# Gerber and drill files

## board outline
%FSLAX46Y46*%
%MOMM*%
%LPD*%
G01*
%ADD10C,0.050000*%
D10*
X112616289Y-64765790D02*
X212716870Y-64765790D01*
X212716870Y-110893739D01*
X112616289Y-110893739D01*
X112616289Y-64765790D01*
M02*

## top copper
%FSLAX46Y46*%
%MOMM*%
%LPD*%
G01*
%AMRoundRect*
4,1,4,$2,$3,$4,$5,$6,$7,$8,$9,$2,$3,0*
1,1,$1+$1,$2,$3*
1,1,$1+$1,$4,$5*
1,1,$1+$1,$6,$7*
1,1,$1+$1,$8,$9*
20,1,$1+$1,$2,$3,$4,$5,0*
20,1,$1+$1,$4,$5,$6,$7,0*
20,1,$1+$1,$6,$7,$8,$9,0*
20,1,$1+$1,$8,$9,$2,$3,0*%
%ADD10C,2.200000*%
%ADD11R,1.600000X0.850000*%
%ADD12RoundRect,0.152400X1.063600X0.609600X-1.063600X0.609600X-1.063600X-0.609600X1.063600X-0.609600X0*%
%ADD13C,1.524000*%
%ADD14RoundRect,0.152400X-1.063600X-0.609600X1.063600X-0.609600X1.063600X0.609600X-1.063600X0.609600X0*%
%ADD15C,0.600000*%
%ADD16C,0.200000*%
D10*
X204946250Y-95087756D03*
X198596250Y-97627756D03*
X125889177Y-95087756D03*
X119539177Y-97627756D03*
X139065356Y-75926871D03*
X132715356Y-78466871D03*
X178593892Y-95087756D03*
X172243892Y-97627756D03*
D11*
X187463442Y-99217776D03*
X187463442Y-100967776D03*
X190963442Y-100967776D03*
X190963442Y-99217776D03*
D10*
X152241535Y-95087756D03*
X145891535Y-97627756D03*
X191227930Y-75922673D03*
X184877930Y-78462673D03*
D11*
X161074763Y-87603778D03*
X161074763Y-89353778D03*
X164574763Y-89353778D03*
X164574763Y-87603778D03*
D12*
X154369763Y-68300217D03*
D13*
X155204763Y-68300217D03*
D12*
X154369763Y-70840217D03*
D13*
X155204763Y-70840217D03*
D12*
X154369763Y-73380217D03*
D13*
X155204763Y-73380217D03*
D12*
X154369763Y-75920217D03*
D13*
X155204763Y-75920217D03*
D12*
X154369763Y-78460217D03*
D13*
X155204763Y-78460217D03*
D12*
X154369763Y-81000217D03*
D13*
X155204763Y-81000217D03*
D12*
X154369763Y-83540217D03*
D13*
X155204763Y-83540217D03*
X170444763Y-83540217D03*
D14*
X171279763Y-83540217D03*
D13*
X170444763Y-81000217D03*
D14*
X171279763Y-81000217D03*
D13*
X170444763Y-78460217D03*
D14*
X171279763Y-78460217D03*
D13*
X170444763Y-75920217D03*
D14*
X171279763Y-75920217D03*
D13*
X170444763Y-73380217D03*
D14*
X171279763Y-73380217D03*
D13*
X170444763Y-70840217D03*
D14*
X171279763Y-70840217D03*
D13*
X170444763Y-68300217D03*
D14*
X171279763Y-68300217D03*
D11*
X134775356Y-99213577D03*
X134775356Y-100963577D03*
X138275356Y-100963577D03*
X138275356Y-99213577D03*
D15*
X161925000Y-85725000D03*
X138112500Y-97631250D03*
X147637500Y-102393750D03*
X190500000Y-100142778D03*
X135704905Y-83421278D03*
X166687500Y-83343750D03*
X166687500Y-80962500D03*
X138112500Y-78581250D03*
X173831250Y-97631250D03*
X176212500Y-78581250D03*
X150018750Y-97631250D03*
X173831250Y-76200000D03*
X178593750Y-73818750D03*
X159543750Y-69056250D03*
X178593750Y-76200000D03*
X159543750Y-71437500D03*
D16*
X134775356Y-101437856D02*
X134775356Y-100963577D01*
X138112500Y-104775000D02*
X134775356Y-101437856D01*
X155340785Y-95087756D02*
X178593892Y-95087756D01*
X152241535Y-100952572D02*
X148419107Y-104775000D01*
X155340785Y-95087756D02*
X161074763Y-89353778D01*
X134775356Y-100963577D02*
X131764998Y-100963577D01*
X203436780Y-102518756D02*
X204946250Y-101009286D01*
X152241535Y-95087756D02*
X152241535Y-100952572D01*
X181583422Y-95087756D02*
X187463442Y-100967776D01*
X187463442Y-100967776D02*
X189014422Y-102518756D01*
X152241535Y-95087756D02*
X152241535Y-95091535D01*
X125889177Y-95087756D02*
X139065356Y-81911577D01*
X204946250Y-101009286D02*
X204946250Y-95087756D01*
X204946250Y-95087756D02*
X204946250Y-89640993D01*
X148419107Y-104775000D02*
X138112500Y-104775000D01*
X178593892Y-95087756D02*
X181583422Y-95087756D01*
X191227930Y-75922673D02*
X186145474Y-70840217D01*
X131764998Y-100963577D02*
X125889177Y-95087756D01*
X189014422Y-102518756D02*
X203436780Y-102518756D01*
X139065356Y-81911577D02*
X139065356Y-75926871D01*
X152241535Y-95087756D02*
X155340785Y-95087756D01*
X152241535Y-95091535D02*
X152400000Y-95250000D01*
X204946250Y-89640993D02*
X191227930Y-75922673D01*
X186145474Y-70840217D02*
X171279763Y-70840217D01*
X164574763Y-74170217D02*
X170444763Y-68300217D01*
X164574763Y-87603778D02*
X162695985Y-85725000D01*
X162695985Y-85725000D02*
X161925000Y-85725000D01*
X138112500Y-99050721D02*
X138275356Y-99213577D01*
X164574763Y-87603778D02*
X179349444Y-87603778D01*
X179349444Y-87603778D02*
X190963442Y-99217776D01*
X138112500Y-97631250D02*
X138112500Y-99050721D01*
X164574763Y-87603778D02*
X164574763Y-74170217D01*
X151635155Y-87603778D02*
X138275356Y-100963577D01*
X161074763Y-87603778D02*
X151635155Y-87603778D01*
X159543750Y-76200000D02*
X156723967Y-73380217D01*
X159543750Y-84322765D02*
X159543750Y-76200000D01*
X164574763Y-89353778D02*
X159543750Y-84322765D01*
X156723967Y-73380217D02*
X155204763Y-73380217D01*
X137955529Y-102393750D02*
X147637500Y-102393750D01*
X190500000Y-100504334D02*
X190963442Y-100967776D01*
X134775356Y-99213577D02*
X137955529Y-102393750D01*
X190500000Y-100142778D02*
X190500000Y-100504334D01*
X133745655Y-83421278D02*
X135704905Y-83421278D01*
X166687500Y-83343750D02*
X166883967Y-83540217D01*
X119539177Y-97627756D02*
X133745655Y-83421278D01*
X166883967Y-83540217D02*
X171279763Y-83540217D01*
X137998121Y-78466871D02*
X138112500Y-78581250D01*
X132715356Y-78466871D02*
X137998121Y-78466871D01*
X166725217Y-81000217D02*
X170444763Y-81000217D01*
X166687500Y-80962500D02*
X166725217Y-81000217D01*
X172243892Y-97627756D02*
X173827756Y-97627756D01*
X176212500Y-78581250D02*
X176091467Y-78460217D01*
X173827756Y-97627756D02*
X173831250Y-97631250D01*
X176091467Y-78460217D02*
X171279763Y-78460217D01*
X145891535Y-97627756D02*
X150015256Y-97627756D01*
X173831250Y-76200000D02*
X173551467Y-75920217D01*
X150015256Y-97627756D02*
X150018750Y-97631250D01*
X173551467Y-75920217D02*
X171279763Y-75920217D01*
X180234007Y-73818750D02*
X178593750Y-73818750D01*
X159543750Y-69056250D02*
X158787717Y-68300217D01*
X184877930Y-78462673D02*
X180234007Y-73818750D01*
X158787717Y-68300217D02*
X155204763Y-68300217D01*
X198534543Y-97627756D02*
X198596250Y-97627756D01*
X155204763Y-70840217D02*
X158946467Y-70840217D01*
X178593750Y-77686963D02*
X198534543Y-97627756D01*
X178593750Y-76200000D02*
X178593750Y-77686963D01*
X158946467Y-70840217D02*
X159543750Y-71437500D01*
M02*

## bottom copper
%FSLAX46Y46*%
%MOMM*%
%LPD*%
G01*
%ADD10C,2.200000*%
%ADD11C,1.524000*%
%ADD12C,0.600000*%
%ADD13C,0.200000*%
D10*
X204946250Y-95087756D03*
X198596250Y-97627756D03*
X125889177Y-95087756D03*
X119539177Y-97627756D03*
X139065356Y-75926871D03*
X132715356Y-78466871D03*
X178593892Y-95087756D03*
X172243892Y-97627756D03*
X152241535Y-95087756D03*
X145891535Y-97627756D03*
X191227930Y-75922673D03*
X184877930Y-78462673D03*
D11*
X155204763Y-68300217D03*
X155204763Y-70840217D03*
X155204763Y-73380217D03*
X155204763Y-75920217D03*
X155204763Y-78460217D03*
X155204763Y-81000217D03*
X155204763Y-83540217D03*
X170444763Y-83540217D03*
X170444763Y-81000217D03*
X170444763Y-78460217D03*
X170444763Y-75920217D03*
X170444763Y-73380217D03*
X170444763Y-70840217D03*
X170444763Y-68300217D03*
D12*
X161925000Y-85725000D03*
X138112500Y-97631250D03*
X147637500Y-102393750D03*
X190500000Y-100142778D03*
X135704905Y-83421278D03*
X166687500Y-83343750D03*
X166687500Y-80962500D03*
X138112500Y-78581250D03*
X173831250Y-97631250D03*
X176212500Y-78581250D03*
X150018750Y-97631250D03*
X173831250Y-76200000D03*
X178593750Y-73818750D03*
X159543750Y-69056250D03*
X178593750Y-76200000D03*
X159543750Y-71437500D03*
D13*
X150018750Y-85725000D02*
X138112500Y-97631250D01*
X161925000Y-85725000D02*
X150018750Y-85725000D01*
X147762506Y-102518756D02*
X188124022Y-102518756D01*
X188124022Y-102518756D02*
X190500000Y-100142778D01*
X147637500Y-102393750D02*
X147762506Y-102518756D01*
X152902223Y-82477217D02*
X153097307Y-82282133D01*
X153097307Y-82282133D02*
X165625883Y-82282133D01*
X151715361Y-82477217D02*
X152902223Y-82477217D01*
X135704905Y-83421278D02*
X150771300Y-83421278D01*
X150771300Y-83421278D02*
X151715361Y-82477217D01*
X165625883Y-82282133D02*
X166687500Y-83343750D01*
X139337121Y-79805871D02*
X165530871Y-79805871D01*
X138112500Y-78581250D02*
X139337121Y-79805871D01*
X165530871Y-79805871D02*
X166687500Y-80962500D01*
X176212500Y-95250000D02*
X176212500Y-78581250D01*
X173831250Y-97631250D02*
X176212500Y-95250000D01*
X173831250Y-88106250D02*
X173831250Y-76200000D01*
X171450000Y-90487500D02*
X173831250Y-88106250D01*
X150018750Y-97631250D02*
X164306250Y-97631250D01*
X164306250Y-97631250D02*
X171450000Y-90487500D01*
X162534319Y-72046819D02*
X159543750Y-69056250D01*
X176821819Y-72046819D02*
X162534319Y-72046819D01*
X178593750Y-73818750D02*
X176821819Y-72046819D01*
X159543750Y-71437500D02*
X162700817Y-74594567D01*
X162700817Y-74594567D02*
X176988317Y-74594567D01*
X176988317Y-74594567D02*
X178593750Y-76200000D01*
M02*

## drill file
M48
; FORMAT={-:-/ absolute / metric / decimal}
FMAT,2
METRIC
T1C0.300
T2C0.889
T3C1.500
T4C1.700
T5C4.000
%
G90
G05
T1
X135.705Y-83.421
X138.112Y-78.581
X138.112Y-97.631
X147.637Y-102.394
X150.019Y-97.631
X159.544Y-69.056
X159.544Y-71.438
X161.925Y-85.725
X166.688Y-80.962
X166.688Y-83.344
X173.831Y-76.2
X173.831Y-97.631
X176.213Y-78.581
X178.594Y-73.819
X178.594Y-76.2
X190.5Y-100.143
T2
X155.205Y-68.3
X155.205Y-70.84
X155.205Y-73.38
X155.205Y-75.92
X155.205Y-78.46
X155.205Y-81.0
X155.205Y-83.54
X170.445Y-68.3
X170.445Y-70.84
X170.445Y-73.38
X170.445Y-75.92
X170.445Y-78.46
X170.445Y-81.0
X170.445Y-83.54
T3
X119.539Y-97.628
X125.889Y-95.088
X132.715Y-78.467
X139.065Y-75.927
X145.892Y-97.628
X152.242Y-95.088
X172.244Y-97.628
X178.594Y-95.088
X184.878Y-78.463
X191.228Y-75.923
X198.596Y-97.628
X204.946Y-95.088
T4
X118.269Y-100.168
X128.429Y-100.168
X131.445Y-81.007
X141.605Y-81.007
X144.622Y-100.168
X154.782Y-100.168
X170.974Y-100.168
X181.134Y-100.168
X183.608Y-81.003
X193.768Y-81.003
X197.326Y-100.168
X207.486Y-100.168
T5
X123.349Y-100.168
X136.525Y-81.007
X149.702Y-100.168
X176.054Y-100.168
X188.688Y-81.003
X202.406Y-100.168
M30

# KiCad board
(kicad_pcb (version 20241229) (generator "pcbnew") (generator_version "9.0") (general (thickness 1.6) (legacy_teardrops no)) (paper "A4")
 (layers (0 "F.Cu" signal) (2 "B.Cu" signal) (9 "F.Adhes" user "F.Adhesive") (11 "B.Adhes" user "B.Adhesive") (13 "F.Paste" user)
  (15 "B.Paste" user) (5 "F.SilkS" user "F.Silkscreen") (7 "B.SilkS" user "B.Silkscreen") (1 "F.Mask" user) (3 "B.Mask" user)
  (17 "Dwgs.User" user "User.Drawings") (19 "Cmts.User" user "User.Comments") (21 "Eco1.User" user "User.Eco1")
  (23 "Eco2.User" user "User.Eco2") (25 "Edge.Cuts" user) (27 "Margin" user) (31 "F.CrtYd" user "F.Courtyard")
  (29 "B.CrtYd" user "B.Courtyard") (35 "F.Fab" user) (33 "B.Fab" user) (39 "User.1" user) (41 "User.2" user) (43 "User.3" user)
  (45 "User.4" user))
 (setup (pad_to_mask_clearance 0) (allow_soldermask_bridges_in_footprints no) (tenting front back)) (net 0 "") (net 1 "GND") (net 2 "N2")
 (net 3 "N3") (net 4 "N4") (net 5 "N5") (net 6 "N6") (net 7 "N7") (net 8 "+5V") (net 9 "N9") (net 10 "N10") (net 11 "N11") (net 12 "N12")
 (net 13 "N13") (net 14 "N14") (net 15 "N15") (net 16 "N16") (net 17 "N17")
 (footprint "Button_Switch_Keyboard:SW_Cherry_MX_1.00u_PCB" (layer "F.Cu") (at 204.94625 95.087756)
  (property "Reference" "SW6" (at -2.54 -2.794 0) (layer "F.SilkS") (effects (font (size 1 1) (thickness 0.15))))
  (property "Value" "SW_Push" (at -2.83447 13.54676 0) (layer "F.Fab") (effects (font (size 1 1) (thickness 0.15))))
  (pad "" np_thru_hole circle (at -7.62 5.08) (size 1.7 1.7) (drill 1.7) (layers "*.Cu" "*.Mask"))
  (pad "" np_thru_hole circle (at -2.54 5.08) (size 4 4) (drill 4) (layers "*.Cu" "*.Mask"))
  (pad "" np_thru_hole circle (at 2.54 5.08) (size 1.7 1.7) (drill 1.7) (layers "*.Cu" "*.Mask"))
  (pad "1" thru_hole circle (at 0 0) (size 2.2 2.2) (drill 1.5) (layers "*.Cu" "*.Mask") (remove_unused_layers no) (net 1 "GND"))
  (pad "2" thru_hole circle (at -6.35 2.54) (size 2.2 2.2) (drill 1.5) (layers "*.Cu" "*.Mask") (remove_unused_layers no) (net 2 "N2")))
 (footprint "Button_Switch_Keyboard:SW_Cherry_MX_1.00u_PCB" (layer "F.Cu") (at 125.889177 95.087756)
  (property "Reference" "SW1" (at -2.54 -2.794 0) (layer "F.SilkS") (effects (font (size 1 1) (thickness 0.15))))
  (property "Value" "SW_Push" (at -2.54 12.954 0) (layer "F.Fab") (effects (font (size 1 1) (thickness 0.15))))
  (pad "" np_thru_hole circle (at -7.62 5.08) (size 1.7 1.7) (drill 1.7) (layers "*.Cu" "*.Mask"))
  (pad "" np_thru_hole circle (at -2.54 5.08) (size 4 4) (drill 4) (layers "*.Cu" "*.Mask"))
  (pad "" np_thru_hole circle (at 2.54 5.08) (size 1.7 1.7) (drill 1.7) (layers "*.Cu" "*.Mask"))
  (pad "1" thru_hole circle (at 0 0) (size 2.2 2.2) (drill 1.5) (layers "*.Cu" "*.Mask") (remove_unused_layers no) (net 1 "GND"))
  (pad "2" thru_hole circle (at -6.35 2.54) (size 2.2 2.2) (drill 1.5) (layers "*.Cu" "*.Mask") (remove_unused_layers no) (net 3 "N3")))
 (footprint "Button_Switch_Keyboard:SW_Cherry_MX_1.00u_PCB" (layer "F.Cu") (at 139.065356 75.926871)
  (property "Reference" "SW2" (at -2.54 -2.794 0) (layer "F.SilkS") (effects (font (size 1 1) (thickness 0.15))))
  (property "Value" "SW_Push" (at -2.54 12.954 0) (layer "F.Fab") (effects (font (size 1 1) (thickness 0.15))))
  (pad "" np_thru_hole circle (at -7.62 5.08) (size 1.7 1.7) (drill 1.7) (layers "*.Cu" "*.Mask"))
  (pad "" np_thru_hole circle (at -2.54 5.08) (size 4 4) (drill 4) (layers "*.Cu" "*.Mask"))
  (pad "" np_thru_hole circle (at 2.54 5.08) (size 1.7 1.7) (drill 1.7) (layers "*.Cu" "*.Mask"))
  (pad "1" thru_hole circle (at 0 0) (size 2.2 2.2) (drill 1.5) (layers "*.Cu" "*.Mask") (remove_unused_layers no) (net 1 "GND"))
  (pad "2" thru_hole circle (at -6.35 2.54) (size 2.2 2.2) (drill 1.5) (layers "*.Cu" "*.Mask") (remove_unused_layers no) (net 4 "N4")))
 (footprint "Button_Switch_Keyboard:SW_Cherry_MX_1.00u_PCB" (layer "F.Cu") (at 178.593892 95.087756)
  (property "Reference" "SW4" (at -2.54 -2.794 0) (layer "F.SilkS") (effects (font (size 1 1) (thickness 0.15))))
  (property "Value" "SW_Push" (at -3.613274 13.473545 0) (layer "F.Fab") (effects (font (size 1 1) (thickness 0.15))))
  (pad "" np_thru_hole circle (at -7.62 5.08) (size 1.7 1.7) (drill 1.7) (layers "*.Cu" "*.Mask"))
  (pad "" np_thru_hole circle (at -2.54 5.08) (size 4 4) (drill 4) (layers "*.Cu" "*.Mask"))
  (pad "" np_thru_hole circle (at 2.54 5.08) (size 1.7 1.7) (drill 1.7) (layers "*.Cu" "*.Mask"))
  (pad "1" thru_hole circle (at 0 0) (size 2.2 2.2) (drill 1.5) (layers "*.Cu" "*.Mask") (remove_unused_layers no) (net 1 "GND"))
  (pad "2" thru_hole circle (at -6.35 2.54) (size 2.2 2.2) (drill 1.5) (layers "*.Cu" "*.Mask") (remove_unused_layers no) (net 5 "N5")))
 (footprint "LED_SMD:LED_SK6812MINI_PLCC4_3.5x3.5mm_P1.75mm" (layer "F.Cu") (at 189.213442 100.092776)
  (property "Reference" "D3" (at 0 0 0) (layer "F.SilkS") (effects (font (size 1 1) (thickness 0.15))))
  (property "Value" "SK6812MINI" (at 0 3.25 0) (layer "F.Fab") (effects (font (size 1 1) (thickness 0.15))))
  (pad "1" smd rect (at -1.75 -0.875) (size 1.6 0.85) (layers "F.Cu" "F.Mask" "F.Paste") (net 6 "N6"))
  (pad "2" smd rect (at -1.75 0.875) (size 1.6 0.85) (layers "F.Cu" "F.Mask" "F.Paste") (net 1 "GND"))
  (pad "3" smd rect (at 1.75 0.875) (size 1.6 0.85) (layers "F.Cu" "F.Mask" "F.Paste") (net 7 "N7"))
  (pad "4" smd rect (at 1.75 -0.875) (size 1.6 0.85) (layers "F.Cu" "F.Mask" "F.Paste") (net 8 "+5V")))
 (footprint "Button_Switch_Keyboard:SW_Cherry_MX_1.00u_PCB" (layer "F.Cu") (at 152.241535 95.087756)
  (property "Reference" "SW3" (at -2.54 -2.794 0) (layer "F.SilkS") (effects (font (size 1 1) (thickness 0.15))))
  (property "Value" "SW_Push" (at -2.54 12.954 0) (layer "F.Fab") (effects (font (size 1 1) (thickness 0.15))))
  (pad "" np_thru_hole circle (at -7.62 5.08) (size 1.7 1.7) (drill 1.7) (layers "*.Cu" "*.Mask"))
  (pad "" np_thru_hole circle (at -2.54 5.08) (size 4 4) (drill 4) (layers "*.Cu" "*.Mask"))
  (pad "" np_thru_hole circle (at 2.54 5.08) (size 1.7 1.7) (drill 1.7) (layers "*.Cu" "*.Mask"))
  (pad "1" thru_hole circle (at 0 0) (size 2.2 2.2) (drill 1.5) (layers "*.Cu" "*.Mask") (remove_unused_layers no) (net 1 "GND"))
  (pad "2" thru_hole circle (at -6.35 2.54) (size 2.2 2.2) (drill 1.5) (layers "*.Cu" "*.Mask") (remove_unused_layers no) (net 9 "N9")))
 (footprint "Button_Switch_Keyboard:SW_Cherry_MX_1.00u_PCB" (layer "F.Cu") (at 191.22793 75.922673)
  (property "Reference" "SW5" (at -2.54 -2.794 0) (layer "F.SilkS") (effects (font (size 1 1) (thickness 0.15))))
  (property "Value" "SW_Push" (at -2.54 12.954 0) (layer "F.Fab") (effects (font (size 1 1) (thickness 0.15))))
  (pad "" np_thru_hole circle (at -7.62 5.08) (size 1.7 1.7) (drill 1.7) (layers "*.Cu" "*.Mask"))
  (pad "" np_thru_hole circle (at -2.54 5.08) (size 4 4) (drill 4) (layers "*.Cu" "*.Mask"))
  (pad "" np_thru_hole circle (at 2.54 5.08) (size 1.7 1.7) (drill 1.7) (layers "*.Cu" "*.Mask"))
  (pad "1" thru_hole circle (at 0 0) (size 2.2 2.2) (drill 1.5) (layers "*.Cu" "*.Mask") (remove_unused_layers no) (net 1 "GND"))
  (pad "2" thru_hole circle (at -6.35 2.54) (size 2.2 2.2) (drill 1.5) (layers "*.Cu" "*.Mask") (remove_unused_layers no) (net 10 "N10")))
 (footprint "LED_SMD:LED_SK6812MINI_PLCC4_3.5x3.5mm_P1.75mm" (layer "F.Cu") (at 162.824763 88.478778)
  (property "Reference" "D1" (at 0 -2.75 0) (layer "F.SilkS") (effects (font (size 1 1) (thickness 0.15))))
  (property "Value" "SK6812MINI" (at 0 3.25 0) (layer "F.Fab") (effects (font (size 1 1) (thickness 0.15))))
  (pad "1" smd rect (at -1.75 -0.875) (size 1.6 0.85) (layers "F.Cu" "F.Mask" "F.Paste") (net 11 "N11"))
  (pad "2" smd rect (at -1.75 0.875) (size 1.6 0.85) (layers "F.Cu" "F.Mask" "F.Paste") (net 1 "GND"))
  (pad "3" smd rect (at 1.75 0.875) (size 1.6 0.85) (layers "F.Cu" "F.Mask" "F.Paste") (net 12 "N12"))
  (pad "4" smd rect (at 1.75 -0.875) (size 1.6 0.85) (layers "F.Cu" "F.Mask" "F.Paste") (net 8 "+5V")))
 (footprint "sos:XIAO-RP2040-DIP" (layer "F.Cu") (at 162.824763 75.920217)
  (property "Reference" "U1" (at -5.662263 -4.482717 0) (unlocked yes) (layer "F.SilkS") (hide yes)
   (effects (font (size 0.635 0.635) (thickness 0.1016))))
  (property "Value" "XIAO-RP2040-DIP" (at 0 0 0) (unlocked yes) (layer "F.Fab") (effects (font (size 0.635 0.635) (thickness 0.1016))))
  (pad "1" smd roundrect (at -8.455 -7.62 180) (size 2.432 1.524) (layers "F.Cu" "F.Mask") (roundrect_rratio 0.1) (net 10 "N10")
   (thermal_bridge_angle 45))
  (pad "1" thru_hole circle (at -7.62 -7.62 180) (size 1.524 1.524) (drill 0.889) (layers "*.Cu" "*.Mask") (remove_unused_layers no)
   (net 10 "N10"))
  (pad "2" smd roundrect (at -8.455 -5.08 180) (size 2.432 1.524) (layers "F.Cu" "F.Mask") (roundrect_rratio 0.1) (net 2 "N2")
   (thermal_bridge_angle 45))
  (pad "2" thru_hole circle (at -7.62 -5.08 180) (size 1.524 1.524) (drill 0.889) (layers "*.Cu" "*.Mask") (remove_unused_layers no)
   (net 2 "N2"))
  (pad "3" smd roundrect (at -8.455 -2.54 180) (size 2.432 1.524) (layers "F.Cu" "F.Mask") (roundrect_rratio 0.1) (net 12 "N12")
   (thermal_bridge_angle 45))
  (pad "3" thru_hole circle (at -7.62 -2.54 180) (size 1.524 1.524) (drill 0.889) (layers "*.Cu" "*.Mask") (remove_unused_layers no)
   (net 12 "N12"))
  (pad "4" smd roundrect (at -8.455 0 180) (size 2.432 1.524) (layers "F.Cu" "F.Mask") (roundrect_rratio 0.1) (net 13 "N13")
   (thermal_bridge_angle 45))
  (pad "4" thru_hole circle (at -7.62 0 180) (size 1.524 1.524) (drill 0.889) (layers "*.Cu" "*.Mask") (remove_unused_layers no)
   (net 13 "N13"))
  (pad "5" smd roundrect (at -8.455 2.54 180) (size 2.432 1.524) (layers "F.Cu" "F.Mask") (roundrect_rratio 0.1) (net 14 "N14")
   (thermal_bridge_angle 45))
  (pad "5" thru_hole circle (at -7.62 2.54 180) (size 1.524 1.524) (drill 0.889) (layers "*.Cu" "*.Mask") (remove_unused_layers no)
   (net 14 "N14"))
  (pad "6" smd roundrect (at -8.455 5.08 180) (size 2.432 1.524) (layers "F.Cu" "F.Mask") (roundrect_rratio 0.1) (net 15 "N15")
   (thermal_bridge_angle 45))
  (pad "6" thru_hole circle (at -7.62 5.08 180) (size 1.524 1.524) (drill 0.889) (layers "*.Cu" "*.Mask") (remove_unused_layers no)
   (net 15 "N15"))
  (pad "7" smd roundrect (at -8.455 7.62 180) (size 2.432 1.524) (layers "F.Cu" "F.Mask") (roundrect_rratio 0.1) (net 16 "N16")
   (thermal_bridge_angle 45))
  (pad "7" thru_hole circle (at -7.62 7.62 180) (size 1.524 1.524) (drill 0.889) (layers "*.Cu" "*.Mask") (remove_unused_layers no)
   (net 16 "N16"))
  (pad "8" thru_hole circle (at 7.62 7.62) (size 1.524 1.524) (drill 0.889) (layers "*.Cu" "*.Mask") (remove_unused_layers no) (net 3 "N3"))
  (pad "8" smd roundrect (at 8.455 7.62) (size 2.432 1.524) (layers "F.Cu" "F.Mask") (roundrect_rratio 0.1) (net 3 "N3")
   (thermal_bridge_angle 45))
  (pad "9" thru_hole circle (at 7.62 5.08) (size 1.524 1.524) (drill 0.889) (layers "*.Cu" "*.Mask") (remove_unused_layers no) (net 4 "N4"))
  (pad "9" smd roundrect (at 8.455 5.08) (size 2.432 1.524) (layers "F.Cu" "F.Mask") (roundrect_rratio 0.1) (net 4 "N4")
   (thermal_bridge_angle 45))
  (pad "10" thru_hole circle (at 7.62 2.54) (size 1.524 1.524) (drill 0.889) (layers "*.Cu" "*.Mask") (remove_unused_layers no) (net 5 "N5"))
  (pad "10" smd roundrect (at 8.455 2.54) (size 2.432 1.524) (layers "F.Cu" "F.Mask") (roundrect_rratio 0.1) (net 5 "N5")
   (thermal_bridge_angle 45))
  (pad "11" thru_hole circle (at 7.62 0) (size 1.524 1.524) (drill 0.889) (layers "*.Cu" "*.Mask") (remove_unused_layers no) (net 9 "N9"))
  (pad "11" smd roundrect (at 8.455 0) (size 2.432 1.524) (layers "F.Cu" "F.Mask") (roundrect_rratio 0.1) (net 9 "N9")
   (thermal_bridge_angle 45))
  (pad "12" thru_hole circle (at 7.62 -2.54) (size 1.524 1.524) (drill 0.889) (layers "*.Cu" "*.Mask") (remove_unused_layers no)
   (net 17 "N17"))
  (pad "12" smd roundrect (at 8.455 -2.54) (size 2.432 1.524) (layers "F.Cu" "F.Mask") (roundrect_rratio 0.1) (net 17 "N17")
   (thermal_bridge_angle 45))
  (pad "13" thru_hole circle (at 7.62 -5.08) (size 1.524 1.524) (drill 0.889) (layers "*.Cu" "*.Mask") (remove_unused_layers no)
   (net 1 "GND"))
  (pad "13" smd roundrect (at 8.455 -5.08) (size 2.432 1.524) (layers "F.Cu" "F.Mask") (roundrect_rratio 0.1) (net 1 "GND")
   (thermal_bridge_angle 45))
  (pad "14" thru_hole circle (at 7.62 -7.62) (size 1.524 1.524) (drill 0.889) (layers "*.Cu" "*.Mask") (remove_unused_layers no)
   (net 8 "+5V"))
  (pad "14" smd roundrect (at 8.455 -7.62) (size 2.432 1.524) (layers "F.Cu" "F.Mask") (roundrect_rratio 0.1) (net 8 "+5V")
   (thermal_bridge_angle 45)))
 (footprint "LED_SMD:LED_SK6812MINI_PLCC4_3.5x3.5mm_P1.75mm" (layer "F.Cu") (at 136.525356 100.088577)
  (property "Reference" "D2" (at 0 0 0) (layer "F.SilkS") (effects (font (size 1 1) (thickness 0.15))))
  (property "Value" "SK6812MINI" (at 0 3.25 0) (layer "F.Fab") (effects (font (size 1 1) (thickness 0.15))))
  (pad "1" smd rect (at -1.75 -0.875) (size 1.6 0.85) (layers "F.Cu" "F.Mask" "F.Paste") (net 7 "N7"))
  (pad "2" smd rect (at -1.75 0.875) (size 1.6 0.85) (layers "F.Cu" "F.Mask" "F.Paste") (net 1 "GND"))
  (pad "3" smd rect (at 1.75 0.875) (size 1.6 0.85) (layers "F.Cu" "F.Mask" "F.Paste") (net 11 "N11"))
  (pad "4" smd rect (at 1.75 -0.875) (size 1.6 0.85) (layers "F.Cu" "F.Mask" "F.Paste") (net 8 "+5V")))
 (gr_rect (start 112.616289 64.76579) (end 212.71687 110.893739) (stroke (width 0.05) (type default)) (fill no) (layer "Edge.Cuts"))
 (segment (start 134.775356 101.437856) (end 134.775356 100.963577) (width 0.2) (layer "F.Cu") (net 1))
 (segment (start 138.1125 104.775) (end 134.775356 101.437856) (width 0.2) (layer "F.Cu") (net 1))
 (segment (start 155.340785 95.087756) (end 178.593892 95.087756) (width 0.2) (layer "F.Cu") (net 1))
 (segment (start 152.241535 100.952572) (end 148.419107 104.775) (width 0.2) (layer "F.Cu") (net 1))
 (segment (start 155.340785 95.087756) (end 161.074763 89.353778) (width 0.2) (layer "F.Cu") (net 1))
 (segment (start 134.775356 100.963577) (end 131.764998 100.963577) (width 0.2) (layer "F.Cu") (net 1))
 (segment (start 203.43678 102.518756) (end 204.94625 101.009286) (width 0.2) (layer "F.Cu") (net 1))
 (segment (start 152.241535 95.087756) (end 152.241535 100.952572) (width 0.2) (layer "F.Cu") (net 1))
 (segment (start 181.583422 95.087756) (end 187.463442 100.967776) (width 0.2) (layer "F.Cu") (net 1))
 (segment (start 187.463442 100.967776) (end 189.014422 102.518756) (width 0.2) (layer "F.Cu") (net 1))
 (segment (start 152.241535 95.087756) (end 152.241535 95.091535) (width 0.2) (layer "F.Cu") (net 1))
 (segment (start 125.889177 95.087756) (end 139.065356 81.911577) (width 0.2) (layer "F.Cu") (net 1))
 (segment (start 204.94625 101.009286) (end 204.94625 95.087756) (width 0.2) (layer "F.Cu") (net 1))
 (segment (start 204.94625 95.087756) (end 204.94625 89.640993) (width 0.2) (layer "F.Cu") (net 1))
 (segment (start 148.419107 104.775) (end 138.1125 104.775) (width 0.2) (layer "F.Cu") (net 1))
 (segment (start 178.593892 95.087756) (end 181.583422 95.087756) (width 0.2) (layer "F.Cu") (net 1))
 (segment (start 191.22793 75.922673) (end 186.145474 70.840217) (width 0.2) (layer "F.Cu") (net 1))
 (segment (start 131.764998 100.963577) (end 125.889177 95.087756) (width 0.2) (layer "F.Cu") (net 1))
 (segment (start 189.014422 102.518756) (end 203.43678 102.518756) (width 0.2) (layer "F.Cu") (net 1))
 (segment (start 139.065356 81.911577) (end 139.065356 75.926871) (width 0.2) (layer "F.Cu") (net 1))
 (segment (start 152.241535 95.087756) (end 155.340785 95.087756) (width 0.2) (layer "F.Cu") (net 1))
 (segment (start 152.241535 95.091535) (end 152.4 95.25) (width 0.2) (layer "F.Cu") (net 1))
 (segment (start 204.94625 89.640993) (end 191.22793 75.922673) (width 0.2) (layer "F.Cu") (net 1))
 (segment (start 186.145474 70.840217) (end 171.279763 70.840217) (width 0.2) (layer "F.Cu") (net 1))
 (segment (start 164.574763 74.170217) (end 170.444763 68.300217) (width 0.2) (layer "F.Cu") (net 8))
 (segment (start 164.574763 87.603778) (end 162.695985 85.725) (width 0.2) (layer "F.Cu") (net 8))
 (segment (start 162.695985 85.725) (end 161.925 85.725) (width 0.2) (layer "F.Cu") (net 8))
 (segment (start 138.1125 99.050721) (end 138.275356 99.213577) (width 0.2) (layer "F.Cu") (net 8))
 (segment (start 164.574763 87.603778) (end 179.349444 87.603778) (width 0.2) (layer "F.Cu") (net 8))
 (segment (start 179.349444 87.603778) (end 190.963442 99.217776) (width 0.2) (layer "F.Cu") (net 8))
 (segment (start 138.1125 97.63125) (end 138.1125 99.050721) (width 0.2) (layer "F.Cu") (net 8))
 (segment (start 164.574763 87.603778) (end 164.574763 74.170217) (width 0.2) (layer "F.Cu") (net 8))
 (via (at 161.925 85.725) (size 0.6) (drill 0.3) (layers "F.Cu" "B.Cu") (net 8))
 (via (at 138.1125 97.63125) (size 0.6) (drill 0.3) (layers "F.Cu" "B.Cu") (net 8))
 (segment (start 150.01875 85.725) (end 138.1125 97.63125) (width 0.2) (layer "B.Cu") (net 8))
 (segment (start 161.925 85.725) (end 150.01875 85.725) (width 0.2) (layer "B.Cu") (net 8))
 (segment (start 151.635155 87.603778) (end 138.275356 100.963577) (width 0.2) (layer "F.Cu") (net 11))
 (segment (start 161.074763 87.603778) (end 151.635155 87.603778) (width 0.2) (layer "F.Cu") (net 11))
 (segment (start 159.54375 76.2) (end 156.723967 73.380217) (width 0.2) (layer "F.Cu") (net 12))
 (segment (start 159.54375 84.322765) (end 159.54375 76.2) (width 0.2) (layer "F.Cu") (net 12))
 (segment (start 164.574763 89.353778) (end 159.54375 84.322765) (width 0.2) (layer "F.Cu") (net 12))
 (segment (start 156.723967 73.380217) (end 155.204763 73.380217) (width 0.2) (layer "F.Cu") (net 12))
 (segment (start 137.955529 102.39375) (end 147.6375 102.39375) (width 0.2) (layer "F.Cu") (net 7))
 (segment (start 190.5 100.504334) (end 190.963442 100.967776) (width 0.2) (layer "F.Cu") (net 7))
 (segment (start 134.775356 99.213577) (end 137.955529 102.39375) (width 0.2) (layer "F.Cu") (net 7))
 (segment (start 190.5 100.142778) (end 190.5 100.504334) (width 0.2) (layer "F.Cu") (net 7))
 (via (at 147.6375 102.39375) (size 0.6) (drill 0.3) (layers "F.Cu" "B.Cu") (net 7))
 (via (at 190.5 100.142778) (size 0.6) (drill 0.3) (layers "F.Cu" "B.Cu") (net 7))
 (segment (start 147.762506 102.518756) (end 188.124022 102.518756) (width 0.2) (layer "B.Cu") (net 7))
 (segment (start 188.124022 102.518756) (end 190.5 100.142778) (width 0.2) (layer "B.Cu") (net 7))
 (segment (start 147.6375 102.39375) (end 147.762506 102.518756) (width 0.2) (layer "B.Cu") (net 7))
 (segment (start 133.745655 83.421278) (end 135.704905 83.421278) (width 0.2) (layer "F.Cu") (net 3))
 (segment (start 166.6875 83.34375) (end 166.883967 83.540217) (width 0.2) (layer "F.Cu") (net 3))
 (segment (start 119.539177 97.627756) (end 133.745655 83.421278) (width 0.2) (layer "F.Cu") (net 3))
 (segment (start 166.883967 83.540217) (end 171.279763 83.540217) (width 0.2) (layer "F.Cu") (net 3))
 (via (at 135.704905 83.421278) (size 0.6) (drill 0.3) (layers "F.Cu" "B.Cu") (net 3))
 (via (at 166.6875 83.34375) (size 0.6) (drill 0.3) (layers "F.Cu" "B.Cu") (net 3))
 (segment (start 152.902223 82.477217) (end 153.097307 82.282133) (width 0.2) (layer "B.Cu") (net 3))
 (segment (start 153.097307 82.282133) (end 165.625883 82.282133) (width 0.2) (layer "B.Cu") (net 3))
 (segment (start 151.715361 82.477217) (end 152.902223 82.477217) (width 0.2) (layer "B.Cu") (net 3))
 (segment (start 135.704905 83.421278) (end 150.7713 83.421278) (width 0.2) (layer "B.Cu") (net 3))
 (segment (start 150.7713 83.421278) (end 151.715361 82.477217) (width 0.2) (layer "B.Cu") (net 3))
 (segment (start 165.625883 82.282133) (end 166.6875 83.34375) (width 0.2) (layer "B.Cu") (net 3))
 (segment (start 137.998121 78.466871) (end 138.1125 78.58125) (width 0.2) (layer "F.Cu") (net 4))
 (segment (start 132.715356 78.466871) (end 137.998121 78.466871) (width 0.2) (layer "F.Cu") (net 4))
 (segment (start 166.725217 81.000217) (end 170.444763 81.000217) (width 0.2) (layer "F.Cu") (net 4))
 (segment (start 166.6875 80.9625) (end 166.725217 81.000217) (width 0.2) (layer "F.Cu") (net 4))
 (via (at 166.6875 80.9625) (size 0.6) (drill 0.3) (layers "F.Cu" "B.Cu") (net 4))
 (via (at 138.1125 78.58125) (size 0.6) (drill 0.3) (layers "F.Cu" "B.Cu") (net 4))
 (segment (start 139.337121 79.805871) (end 165.530871 79.805871) (width 0.2) (layer "B.Cu") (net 4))
 (segment (start 138.1125 78.58125) (end 139.337121 79.805871) (width 0.2) (layer "B.Cu") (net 4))
 (segment (start 165.530871 79.805871) (end 166.6875 80.9625) (width 0.2) (layer "B.Cu") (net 4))
 (segment (start 172.243892 97.627756) (end 173.827756 97.627756) (width 0.2) (layer "F.Cu") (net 5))
 (segment (start 176.2125 78.58125) (end 176.091467 78.460217) (width 0.2) (layer "F.Cu") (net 5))
 (segment (start 173.827756 97.627756) (end 173.83125 97.63125) (width 0.2) (layer "F.Cu") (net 5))
 (segment (start 176.091467 78.460217) (end 171.279763 78.460217) (width 0.2) (layer "F.Cu") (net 5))
 (via (at 173.83125 97.63125) (size 0.6) (drill 0.3) (layers "F.Cu" "B.Cu") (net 5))
 (via (at 176.2125 78.58125) (size 0.6) (drill 0.3) (layers "F.Cu" "B.Cu") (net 5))
 (segment (start 176.2125 95.25) (end 176.2125 78.58125) (width 0.2) (layer "B.Cu") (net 5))
 (segment (start 173.83125 97.63125) (end 176.2125 95.25) (width 0.2) (layer "B.Cu") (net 5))
 (segment (start 145.891535 97.627756) (end 150.015256 97.627756) (width 0.2) (layer "F.Cu") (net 9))
 (segment (start 173.83125 76.2) (end 173.551467 75.920217) (width 0.2) (layer "F.Cu") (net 9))
 (segment (start 150.015256 97.627756) (end 150.01875 97.63125) (width 0.2) (layer "F.Cu") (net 9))
 (segment (start 173.551467 75.920217) (end 171.279763 75.920217) (width 0.2) (layer "F.Cu") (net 9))
 (via (at 150.01875 97.63125) (size 0.6) (drill 0.3) (layers "F.Cu" "B.Cu") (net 9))
 (via (at 173.83125 76.2) (size 0.6) (drill 0.3) (layers "F.Cu" "B.Cu") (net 9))
 (segment (start 173.83125 88.10625) (end 173.83125 76.2) (width 0.2) (layer "B.Cu") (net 9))
 (segment (start 171.45 90.4875) (end 173.83125 88.10625) (width 0.2) (layer "B.Cu") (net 9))
 (segment (start 150.01875 97.63125) (end 164.30625 97.63125) (width 0.2) (layer "B.Cu") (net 9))
 (segment (start 164.30625 97.63125) (end 171.45 90.4875) (width 0.2) (layer "B.Cu") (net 9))
 (segment (start 180.234007 73.81875) (end 178.59375 73.81875) (width 0.2) (layer "F.Cu") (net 10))
 (segment (start 159.54375 69.05625) (end 158.787717 68.300217) (width 0.2) (layer "F.Cu") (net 10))
 (segment (start 184.87793 78.462673) (end 180.234007 73.81875) (width 0.2) (layer "F.Cu") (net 10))
 (segment (start 158.787717 68.300217) (end 155.204763 68.300217) (width 0.2) (layer "F.Cu") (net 10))
 (via (at 178.59375 73.81875) (size 0.6) (drill 0.3) (layers "F.Cu" "B.Cu") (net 10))
 (via (at 159.54375 69.05625) (size 0.6) (drill 0.3) (layers "F.Cu" "B.Cu") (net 10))
 (segment (start 162.534319 72.046819) (end 159.54375 69.05625) (width 0.2) (layer "B.Cu") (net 10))
 (segment (start 176.821819 72.046819) (end 162.534319 72.046819) (width 0.2) (layer "B.Cu") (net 10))
 (segment (start 178.59375 73.81875) (end 176.821819 72.046819) (width 0.2) (layer "B.Cu") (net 10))
 (segment (start 198.534543 97.627756) (end 198.59625 97.627756) (width 0.2) (layer "F.Cu") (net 2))
 (segment (start 155.204763 70.840217) (end 158.946467 70.840217) (width 0.2) (layer "F.Cu") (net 2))
 (segment (start 178.59375 77.686963) (end 198.534543 97.627756) (width 0.2) (layer "F.Cu") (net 2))
 (segment (start 178.59375 76.2) (end 178.59375 77.686963) (width 0.2) (layer "F.Cu") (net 2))
 (segment (start 158.946467 70.840217) (end 159.54375 71.4375) (width 0.2) (layer "F.Cu") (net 2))
 (via (at 178.59375 76.2) (size 0.6) (drill 0.3) (layers "F.Cu" "B.Cu") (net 2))
 (via (at 159.54375 71.4375) (size 0.6) (drill 0.3) (layers "F.Cu" "B.Cu") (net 2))
 (segment (start 159.54375 71.4375) (end 162.700817 74.594567) (width 0.2) (layer "B.Cu") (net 2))
 (segment (start 162.700817 74.594567) (end 176.988317 74.594567) (width 0.2) (layer "B.Cu") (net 2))
 (segment (start 176.988317 74.594567) (end 178.59375 76.2) (width 0.2) (layer "B.Cu") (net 2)))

